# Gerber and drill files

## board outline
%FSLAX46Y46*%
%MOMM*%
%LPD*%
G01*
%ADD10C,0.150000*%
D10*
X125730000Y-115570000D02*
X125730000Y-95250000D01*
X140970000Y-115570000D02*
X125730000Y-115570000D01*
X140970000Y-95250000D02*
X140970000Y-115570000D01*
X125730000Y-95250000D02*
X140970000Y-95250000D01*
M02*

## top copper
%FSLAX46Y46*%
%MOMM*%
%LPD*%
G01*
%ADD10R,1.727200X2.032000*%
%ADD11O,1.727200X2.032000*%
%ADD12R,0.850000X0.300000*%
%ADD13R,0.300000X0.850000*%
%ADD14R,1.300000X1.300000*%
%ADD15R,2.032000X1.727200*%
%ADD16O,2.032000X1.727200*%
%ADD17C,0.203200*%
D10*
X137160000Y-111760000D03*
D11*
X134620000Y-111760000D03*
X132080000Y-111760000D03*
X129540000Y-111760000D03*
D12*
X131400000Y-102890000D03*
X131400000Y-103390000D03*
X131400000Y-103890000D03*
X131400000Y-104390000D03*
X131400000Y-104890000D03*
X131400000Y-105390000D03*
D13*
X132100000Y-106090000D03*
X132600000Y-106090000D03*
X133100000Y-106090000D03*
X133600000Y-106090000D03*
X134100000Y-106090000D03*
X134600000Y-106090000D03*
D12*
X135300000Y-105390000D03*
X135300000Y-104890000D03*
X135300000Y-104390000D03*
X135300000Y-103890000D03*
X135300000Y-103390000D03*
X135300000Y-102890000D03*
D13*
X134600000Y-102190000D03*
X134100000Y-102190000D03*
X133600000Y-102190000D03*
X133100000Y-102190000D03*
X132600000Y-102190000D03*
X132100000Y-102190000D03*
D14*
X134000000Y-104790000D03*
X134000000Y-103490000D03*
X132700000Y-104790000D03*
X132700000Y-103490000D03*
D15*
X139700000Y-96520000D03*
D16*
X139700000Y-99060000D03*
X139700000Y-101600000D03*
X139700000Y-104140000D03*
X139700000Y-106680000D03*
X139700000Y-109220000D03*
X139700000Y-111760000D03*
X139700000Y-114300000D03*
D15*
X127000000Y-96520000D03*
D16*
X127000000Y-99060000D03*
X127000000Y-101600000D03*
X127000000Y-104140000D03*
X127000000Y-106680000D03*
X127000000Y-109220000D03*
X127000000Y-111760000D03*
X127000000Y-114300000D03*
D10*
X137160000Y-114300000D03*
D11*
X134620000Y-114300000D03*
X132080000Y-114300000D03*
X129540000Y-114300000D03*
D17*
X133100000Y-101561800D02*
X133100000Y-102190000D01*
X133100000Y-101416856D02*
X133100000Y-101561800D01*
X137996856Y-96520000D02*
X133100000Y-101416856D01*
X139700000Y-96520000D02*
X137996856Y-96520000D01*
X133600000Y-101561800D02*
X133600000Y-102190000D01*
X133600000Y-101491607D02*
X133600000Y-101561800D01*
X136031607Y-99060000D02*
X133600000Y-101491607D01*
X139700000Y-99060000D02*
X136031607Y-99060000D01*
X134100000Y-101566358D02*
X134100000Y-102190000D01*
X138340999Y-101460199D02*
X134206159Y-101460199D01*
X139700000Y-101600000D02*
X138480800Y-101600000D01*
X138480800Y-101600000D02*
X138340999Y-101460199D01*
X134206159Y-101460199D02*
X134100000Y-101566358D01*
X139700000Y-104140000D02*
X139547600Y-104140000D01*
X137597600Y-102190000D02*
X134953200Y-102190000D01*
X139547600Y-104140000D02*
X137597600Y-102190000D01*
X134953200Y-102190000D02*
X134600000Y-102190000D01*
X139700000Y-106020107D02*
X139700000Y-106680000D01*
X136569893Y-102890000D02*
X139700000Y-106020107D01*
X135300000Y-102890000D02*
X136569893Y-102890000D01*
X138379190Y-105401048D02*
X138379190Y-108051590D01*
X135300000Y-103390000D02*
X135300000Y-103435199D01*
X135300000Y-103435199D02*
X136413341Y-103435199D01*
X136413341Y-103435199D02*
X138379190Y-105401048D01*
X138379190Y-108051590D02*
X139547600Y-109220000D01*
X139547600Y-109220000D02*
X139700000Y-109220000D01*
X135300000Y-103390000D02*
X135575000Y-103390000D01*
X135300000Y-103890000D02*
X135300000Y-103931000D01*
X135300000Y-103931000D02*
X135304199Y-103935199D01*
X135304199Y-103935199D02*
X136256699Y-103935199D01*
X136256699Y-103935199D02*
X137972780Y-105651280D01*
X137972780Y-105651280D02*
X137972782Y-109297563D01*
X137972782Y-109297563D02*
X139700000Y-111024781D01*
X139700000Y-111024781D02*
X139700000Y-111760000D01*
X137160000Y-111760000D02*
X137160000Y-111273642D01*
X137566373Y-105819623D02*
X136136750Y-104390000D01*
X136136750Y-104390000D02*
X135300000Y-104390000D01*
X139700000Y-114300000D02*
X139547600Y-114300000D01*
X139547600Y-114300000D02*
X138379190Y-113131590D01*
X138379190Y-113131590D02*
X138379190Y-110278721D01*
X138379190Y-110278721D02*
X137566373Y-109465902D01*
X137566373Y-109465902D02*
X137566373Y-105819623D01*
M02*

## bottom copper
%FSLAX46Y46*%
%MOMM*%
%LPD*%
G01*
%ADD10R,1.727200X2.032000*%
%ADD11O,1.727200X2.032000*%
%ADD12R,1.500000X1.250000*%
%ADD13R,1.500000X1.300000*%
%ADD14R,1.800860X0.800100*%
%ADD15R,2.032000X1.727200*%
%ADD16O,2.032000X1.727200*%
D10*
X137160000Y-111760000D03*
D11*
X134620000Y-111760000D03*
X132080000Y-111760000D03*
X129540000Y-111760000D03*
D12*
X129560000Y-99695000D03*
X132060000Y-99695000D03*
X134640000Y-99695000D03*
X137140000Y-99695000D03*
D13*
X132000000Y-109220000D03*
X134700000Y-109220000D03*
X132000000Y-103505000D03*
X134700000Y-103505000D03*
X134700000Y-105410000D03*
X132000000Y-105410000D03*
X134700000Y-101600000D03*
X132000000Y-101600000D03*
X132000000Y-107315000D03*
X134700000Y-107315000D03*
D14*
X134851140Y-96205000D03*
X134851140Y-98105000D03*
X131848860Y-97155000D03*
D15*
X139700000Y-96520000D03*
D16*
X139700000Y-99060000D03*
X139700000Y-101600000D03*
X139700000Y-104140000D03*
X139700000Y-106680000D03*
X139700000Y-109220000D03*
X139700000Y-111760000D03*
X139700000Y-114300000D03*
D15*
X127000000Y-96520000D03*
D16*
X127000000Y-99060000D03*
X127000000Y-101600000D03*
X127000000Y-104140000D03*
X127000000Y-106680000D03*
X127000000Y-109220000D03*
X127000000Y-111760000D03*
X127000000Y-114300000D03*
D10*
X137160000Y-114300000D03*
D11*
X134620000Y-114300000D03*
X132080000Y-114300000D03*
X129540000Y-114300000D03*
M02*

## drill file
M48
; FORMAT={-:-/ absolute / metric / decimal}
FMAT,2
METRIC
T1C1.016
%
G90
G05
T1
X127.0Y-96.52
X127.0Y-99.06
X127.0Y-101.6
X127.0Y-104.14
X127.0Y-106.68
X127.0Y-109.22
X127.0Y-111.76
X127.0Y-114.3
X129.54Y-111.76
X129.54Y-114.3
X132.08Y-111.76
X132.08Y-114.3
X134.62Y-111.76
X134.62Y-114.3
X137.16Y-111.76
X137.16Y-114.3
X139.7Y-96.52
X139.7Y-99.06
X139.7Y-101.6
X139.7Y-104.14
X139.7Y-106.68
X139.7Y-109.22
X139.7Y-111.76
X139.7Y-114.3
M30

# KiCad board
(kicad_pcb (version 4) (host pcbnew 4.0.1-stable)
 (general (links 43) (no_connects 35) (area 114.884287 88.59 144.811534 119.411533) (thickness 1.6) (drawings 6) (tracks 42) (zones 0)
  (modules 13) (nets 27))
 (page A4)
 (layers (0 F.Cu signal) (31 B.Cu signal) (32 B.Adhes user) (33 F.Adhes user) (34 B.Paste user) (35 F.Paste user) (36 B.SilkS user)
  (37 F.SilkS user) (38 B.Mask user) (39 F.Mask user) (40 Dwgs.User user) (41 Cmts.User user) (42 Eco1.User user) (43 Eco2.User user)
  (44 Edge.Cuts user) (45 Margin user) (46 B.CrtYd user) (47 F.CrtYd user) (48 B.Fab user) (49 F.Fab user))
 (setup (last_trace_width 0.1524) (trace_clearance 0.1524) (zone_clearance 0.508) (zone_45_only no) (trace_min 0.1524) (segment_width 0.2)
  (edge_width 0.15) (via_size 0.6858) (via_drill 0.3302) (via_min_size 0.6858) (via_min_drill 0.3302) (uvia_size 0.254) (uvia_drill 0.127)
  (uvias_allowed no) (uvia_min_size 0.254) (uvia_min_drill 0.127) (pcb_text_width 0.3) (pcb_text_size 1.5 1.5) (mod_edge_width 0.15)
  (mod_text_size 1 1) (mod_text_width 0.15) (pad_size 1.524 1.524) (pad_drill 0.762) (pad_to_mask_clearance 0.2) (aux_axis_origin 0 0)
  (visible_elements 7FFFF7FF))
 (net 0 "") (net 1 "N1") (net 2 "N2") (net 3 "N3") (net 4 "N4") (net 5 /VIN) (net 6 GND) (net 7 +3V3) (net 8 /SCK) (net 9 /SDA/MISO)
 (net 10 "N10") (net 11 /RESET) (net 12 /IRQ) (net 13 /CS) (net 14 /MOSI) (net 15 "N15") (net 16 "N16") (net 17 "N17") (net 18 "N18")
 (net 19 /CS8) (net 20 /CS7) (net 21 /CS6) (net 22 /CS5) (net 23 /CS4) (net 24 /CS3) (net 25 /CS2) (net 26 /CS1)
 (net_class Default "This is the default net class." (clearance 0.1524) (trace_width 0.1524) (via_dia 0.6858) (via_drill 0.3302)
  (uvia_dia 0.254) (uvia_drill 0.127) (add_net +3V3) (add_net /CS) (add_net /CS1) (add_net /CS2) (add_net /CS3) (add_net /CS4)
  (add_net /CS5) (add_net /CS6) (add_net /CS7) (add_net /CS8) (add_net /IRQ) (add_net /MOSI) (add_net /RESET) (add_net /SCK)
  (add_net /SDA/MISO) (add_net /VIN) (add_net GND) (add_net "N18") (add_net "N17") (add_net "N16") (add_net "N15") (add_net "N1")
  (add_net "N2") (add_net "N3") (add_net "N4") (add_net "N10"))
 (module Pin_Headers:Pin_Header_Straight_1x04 (layer F.Cu) (at 137.16 111.76 270)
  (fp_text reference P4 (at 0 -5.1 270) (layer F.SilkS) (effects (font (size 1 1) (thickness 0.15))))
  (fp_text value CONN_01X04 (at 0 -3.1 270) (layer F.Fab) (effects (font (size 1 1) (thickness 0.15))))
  (pad 1 thru_hole rect (at 0 0 270) (size 2.032 1.7272) (drill 1.016) (layers *.Cu *.Mask F.SilkS) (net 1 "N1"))
  (pad 2 thru_hole oval (at 0 2.54 270) (size 2.032 1.7272) (drill 1.016) (layers *.Cu *.Mask F.SilkS) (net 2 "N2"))
  (pad 3 thru_hole oval (at 0 5.08 270) (size 2.032 1.7272) (drill 1.016) (layers *.Cu *.Mask F.SilkS) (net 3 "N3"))
  (pad 4 thru_hole oval (at 0 7.62 270) (size 2.032 1.7272) (drill 1.016) (layers *.Cu *.Mask F.SilkS) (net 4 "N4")))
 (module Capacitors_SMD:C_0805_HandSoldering (layer B.Cu) (at 130.81 99.695)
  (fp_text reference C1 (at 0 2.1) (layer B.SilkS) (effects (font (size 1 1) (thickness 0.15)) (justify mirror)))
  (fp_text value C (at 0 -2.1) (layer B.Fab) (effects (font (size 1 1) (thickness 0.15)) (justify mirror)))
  (pad 1 smd rect (at -1.25 0) (size 1.5 1.25) (layers B.Cu B.Paste B.Mask) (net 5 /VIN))
  (pad 2 smd rect (at 1.25 0) (size 1.5 1.25) (layers B.Cu B.Paste B.Mask) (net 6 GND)))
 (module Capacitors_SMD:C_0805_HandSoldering (layer B.Cu) (at 135.89 99.695)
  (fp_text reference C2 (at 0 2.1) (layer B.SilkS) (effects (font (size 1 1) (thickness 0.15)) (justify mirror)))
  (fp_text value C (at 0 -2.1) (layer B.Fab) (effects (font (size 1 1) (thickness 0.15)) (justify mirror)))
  (pad 1 smd rect (at -1.25 0) (size 1.5 1.25) (layers B.Cu B.Paste B.Mask) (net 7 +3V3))
  (pad 2 smd rect (at 1.25 0) (size 1.5 1.25) (layers B.Cu B.Paste B.Mask) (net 6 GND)))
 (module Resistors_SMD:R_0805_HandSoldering (layer B.Cu) (at 133.35 109.22)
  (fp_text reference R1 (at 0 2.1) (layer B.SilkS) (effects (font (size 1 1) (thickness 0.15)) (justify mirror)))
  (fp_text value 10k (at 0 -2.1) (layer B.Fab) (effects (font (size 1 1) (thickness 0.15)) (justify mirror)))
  (pad 1 smd rect (at -1.35 0) (size 1.5 1.3) (layers B.Cu B.Paste B.Mask) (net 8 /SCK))
  (pad 2 smd rect (at 1.35 0) (size 1.5 1.3) (layers B.Cu B.Paste B.Mask) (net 7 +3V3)))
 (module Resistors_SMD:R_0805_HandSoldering (layer B.Cu) (at 133.35 103.505)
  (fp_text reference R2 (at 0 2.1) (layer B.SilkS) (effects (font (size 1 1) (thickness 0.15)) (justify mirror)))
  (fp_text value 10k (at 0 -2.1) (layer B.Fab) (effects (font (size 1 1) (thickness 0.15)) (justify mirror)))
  (pad 1 smd rect (at -1.35 0) (size 1.5 1.3) (layers B.Cu B.Paste B.Mask) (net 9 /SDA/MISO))
  (pad 2 smd rect (at 1.35 0) (size 1.5 1.3) (layers B.Cu B.Paste B.Mask) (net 7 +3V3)))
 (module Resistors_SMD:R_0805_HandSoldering (layer B.Cu) (at 133.35 105.41 180)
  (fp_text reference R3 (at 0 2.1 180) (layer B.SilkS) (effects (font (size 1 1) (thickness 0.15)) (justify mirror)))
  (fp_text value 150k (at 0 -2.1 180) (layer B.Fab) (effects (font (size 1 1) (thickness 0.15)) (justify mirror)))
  (pad 1 smd rect (at -1.35 0 180) (size 1.5 1.3) (layers B.Cu B.Paste B.Mask) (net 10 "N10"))
  (pad 2 smd rect (at 1.35 0 180) (size 1.5 1.3) (layers B.Cu B.Paste B.Mask) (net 6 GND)))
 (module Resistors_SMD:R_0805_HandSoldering (layer B.Cu) (at 133.35 101.6 180)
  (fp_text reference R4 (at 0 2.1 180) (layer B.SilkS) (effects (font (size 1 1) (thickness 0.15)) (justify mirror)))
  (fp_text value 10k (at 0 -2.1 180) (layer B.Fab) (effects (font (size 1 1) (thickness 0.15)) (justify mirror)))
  (pad 1 smd rect (at -1.35 0 180) (size 1.5 1.3) (layers B.Cu B.Paste B.Mask) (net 6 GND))
  (pad 2 smd rect (at 1.35 0 180) (size 1.5 1.3) (layers B.Cu B.Paste B.Mask) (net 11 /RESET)))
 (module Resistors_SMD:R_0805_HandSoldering (layer B.Cu) (at 133.35 107.315)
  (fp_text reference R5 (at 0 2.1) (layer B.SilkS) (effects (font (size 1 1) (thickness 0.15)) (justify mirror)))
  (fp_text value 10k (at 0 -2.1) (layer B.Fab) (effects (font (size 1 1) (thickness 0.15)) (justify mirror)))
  (pad 1 smd rect (at -1.35 0) (size 1.5 1.3) (layers B.Cu B.Paste B.Mask) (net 7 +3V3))
  (pad 2 smd rect (at 1.35 0) (size 1.5 1.3) (layers B.Cu B.Paste B.Mask) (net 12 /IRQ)))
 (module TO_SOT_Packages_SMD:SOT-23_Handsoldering (layer B.Cu) (at 133.35 97.155 270)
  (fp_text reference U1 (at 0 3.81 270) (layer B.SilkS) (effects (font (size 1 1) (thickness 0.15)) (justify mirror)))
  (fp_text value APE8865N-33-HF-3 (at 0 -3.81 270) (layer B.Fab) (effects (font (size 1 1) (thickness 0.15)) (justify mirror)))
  (pad 1 smd rect (at -0.95 -1.50114 270) (size 0.8001 1.80086) (layers B.Cu B.Paste B.Mask) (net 6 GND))
  (pad 2 smd rect (at 0.95 -1.50114 270) (size 0.8001 1.80086) (layers B.Cu B.Paste B.Mask) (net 7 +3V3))
  (pad 3 smd rect (at 0 1.50114 270) (size 0.8001 1.80086) (layers B.Cu B.Paste B.Mask) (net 5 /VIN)))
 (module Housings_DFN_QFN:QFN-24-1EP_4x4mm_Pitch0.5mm (layer F.Cu) (at 133.35 104.14)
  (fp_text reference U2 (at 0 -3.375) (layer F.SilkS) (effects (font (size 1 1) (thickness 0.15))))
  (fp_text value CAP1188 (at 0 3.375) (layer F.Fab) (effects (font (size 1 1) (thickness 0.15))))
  (pad 1 smd rect (at -1.95 -1.25) (size 0.85 0.3) (layers F.Cu F.Paste F.Mask) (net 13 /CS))
  (pad 2 smd rect (at -1.95 -0.75) (size 0.85 0.3) (layers F.Cu F.Paste F.Mask) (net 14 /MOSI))
  (pad 3 smd rect (at -1.95 -0.25) (size 0.85 0.3) (layers F.Cu F.Paste F.Mask) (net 9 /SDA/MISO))
  (pad 4 smd rect (at -1.95 0.25) (size 0.85 0.3) (layers F.Cu F.Paste F.Mask) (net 8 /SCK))
  (pad 5 smd rect (at -1.95 0.75) (size 0.85 0.3) (layers F.Cu F.Paste F.Mask) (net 4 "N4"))
  (pad 6 smd rect (at -1.95 1.25) (size 0.85 0.3) (layers F.Cu F.Paste F.Mask) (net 3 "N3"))
  (pad 7 smd rect (at -1.25 1.95 90) (size 0.85 0.3) (layers F.Cu F.Paste F.Mask) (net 2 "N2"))
  (pad 8 smd rect (at -0.75 1.95 90) (size 0.85 0.3) (layers F.Cu F.Paste F.Mask) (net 1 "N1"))
  (pad 9 smd rect (at -0.25 1.95 90) (size 0.85 0.3) (layers F.Cu F.Paste F.Mask) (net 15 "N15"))
  (pad 10 smd rect (at 0.25 1.95 90) (size 0.85 0.3) (layers F.Cu F.Paste F.Mask) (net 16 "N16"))
  (pad 11 smd rect (at 0.75 1.95 90) (size 0.85 0.3) (layers F.Cu F.Paste F.Mask) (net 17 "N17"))
  (pad 12 smd rect (at 1.25 1.95 90) (size 0.85 0.3) (layers F.Cu F.Paste F.Mask) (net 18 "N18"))
  (pad 13 smd rect (at 1.95 1.25) (size 0.85 0.3) (layers F.Cu F.Paste F.Mask) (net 12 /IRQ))
  (pad 14 smd rect (at 1.95 0.75) (size 0.85 0.3) (layers F.Cu F.Paste F.Mask) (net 10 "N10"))
  (pad 15 smd rect (at 1.95 0.25) (size 0.85 0.3) (layers F.Cu F.Paste F.Mask) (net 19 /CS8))
  (pad 16 smd rect (at 1.95 -0.25) (size 0.85 0.3) (layers F.Cu F.Paste F.Mask) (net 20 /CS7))
  (pad 17 smd rect (at 1.95 -0.75) (size 0.85 0.3) (layers F.Cu F.Paste F.Mask) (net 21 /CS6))
  (pad 18 smd rect (at 1.95 -1.25) (size 0.85 0.3) (layers F.Cu F.Paste F.Mask) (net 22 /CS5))
  (pad 19 smd rect (at 1.25 -1.95 90) (size 0.85 0.3) (layers F.Cu F.Paste F.Mask) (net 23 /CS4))
  (pad 20 smd rect (at 0.75 -1.95 90) (size 0.85 0.3) (layers F.Cu F.Paste F.Mask) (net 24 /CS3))
  (pad 21 smd rect (at 0.25 -1.95 90) (size 0.85 0.3) (layers F.Cu F.Paste F.Mask) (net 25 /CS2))
  (pad 22 smd rect (at -0.25 -1.95 90) (size 0.85 0.3) (layers F.Cu F.Paste F.Mask) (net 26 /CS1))
  (pad 23 smd rect (at -0.75 -1.95 90) (size 0.85 0.3) (layers F.Cu F.Paste F.Mask) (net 7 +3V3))
  (pad 24 smd rect (at -1.25 -1.95 90) (size 0.85 0.3) (layers F.Cu F.Paste F.Mask) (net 11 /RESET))
  (pad 25 smd rect (at 0.65 0.65) (size 1.3 1.3) (layers F.Cu F.Paste F.Mask) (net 6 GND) (solder_paste_margin_ratio -0.2))
  (pad 25 smd rect (at 0.65 -0.65) (size 1.3 1.3) (layers F.Cu F.Paste F.Mask) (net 6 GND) (solder_paste_margin_ratio -0.2))
  (pad 25 smd rect (at -0.65 0.65) (size 1.3 1.3) (layers F.Cu F.Paste F.Mask) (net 6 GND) (solder_paste_margin_ratio -0.2))
  (pad 25 smd rect (at -0.65 -0.65) (size 1.3 1.3) (layers F.Cu F.Paste F.Mask) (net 6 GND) (solder_paste_margin_ratio -0.2)))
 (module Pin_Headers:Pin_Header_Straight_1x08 (layer B.Cu) (at 139.7 96.52 180)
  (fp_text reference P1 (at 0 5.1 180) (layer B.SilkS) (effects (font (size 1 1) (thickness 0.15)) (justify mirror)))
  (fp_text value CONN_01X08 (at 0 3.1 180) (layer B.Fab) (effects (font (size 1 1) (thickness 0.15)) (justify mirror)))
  (pad 1 thru_hole rect (at 0 0 180) (size 2.032 1.7272) (drill 1.016) (layers *.Cu *.Mask B.SilkS) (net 26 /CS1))
  (pad 2 thru_hole oval (at 0 -2.54 180) (size 2.032 1.7272) (drill 1.016) (layers *.Cu *.Mask B.SilkS) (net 25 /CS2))
  (pad 3 thru_hole oval (at 0 -5.08 180) (size 2.032 1.7272) (drill 1.016) (layers *.Cu *.Mask B.SilkS) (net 24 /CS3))
  (pad 4 thru_hole oval (at 0 -7.62 180) (size 2.032 1.7272) (drill 1.016) (layers *.Cu *.Mask B.SilkS) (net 23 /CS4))
  (pad 5 thru_hole oval (at 0 -10.16 180) (size 2.032 1.7272) (drill 1.016) (layers *.Cu *.Mask B.SilkS) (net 22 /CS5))
  (pad 6 thru_hole oval (at 0 -12.7 180) (size 2.032 1.7272) (drill 1.016) (layers *.Cu *.Mask B.SilkS) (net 21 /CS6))
  (pad 7 thru_hole oval (at 0 -15.24 180) (size 2.032 1.7272) (drill 1.016) (layers *.Cu *.Mask B.SilkS) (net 20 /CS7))
  (pad 8 thru_hole oval (at 0 -17.78 180) (size 2.032 1.7272) (drill 1.016) (layers *.Cu *.Mask B.SilkS) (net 19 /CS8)))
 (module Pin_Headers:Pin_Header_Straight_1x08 (layer B.Cu) (at 127 96.52 180)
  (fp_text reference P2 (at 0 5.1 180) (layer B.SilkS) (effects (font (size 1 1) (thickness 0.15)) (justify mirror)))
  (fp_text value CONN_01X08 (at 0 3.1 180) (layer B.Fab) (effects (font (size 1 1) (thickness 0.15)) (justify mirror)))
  (pad 1 thru_hole rect (at 0 0 180) (size 2.032 1.7272) (drill 1.016) (layers *.Cu *.Mask B.SilkS) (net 9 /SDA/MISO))
  (pad 2 thru_hole oval (at 0 -2.54 180) (size 2.032 1.7272) (drill 1.016) (layers *.Cu *.Mask B.SilkS) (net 8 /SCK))
  (pad 3 thru_hole oval (at 0 -5.08 180) (size 2.032 1.7272) (drill 1.016) (layers *.Cu *.Mask B.SilkS) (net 5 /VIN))
  (pad 4 thru_hole oval (at 0 -7.62 180) (size 2.032 1.7272) (drill 1.016) (layers *.Cu *.Mask B.SilkS) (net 6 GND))
  (pad 5 thru_hole oval (at 0 -10.16 180) (size 2.032 1.7272) (drill 1.016) (layers *.Cu *.Mask B.SilkS) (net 14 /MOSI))
  (pad 6 thru_hole oval (at 0 -12.7 180) (size 2.032 1.7272) (drill 1.016) (layers *.Cu *.Mask B.SilkS) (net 13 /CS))
  (pad 7 thru_hole oval (at 0 -15.24 180) (size 2.032 1.7272) (drill 1.016) (layers *.Cu *.Mask B.SilkS) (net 11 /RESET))
  (pad 8 thru_hole oval (at 0 -17.78 180) (size 2.032 1.7272) (drill 1.016) (layers *.Cu *.Mask B.SilkS) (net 12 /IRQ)))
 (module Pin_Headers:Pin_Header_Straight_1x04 (layer F.Cu) (at 137.16 114.3 270)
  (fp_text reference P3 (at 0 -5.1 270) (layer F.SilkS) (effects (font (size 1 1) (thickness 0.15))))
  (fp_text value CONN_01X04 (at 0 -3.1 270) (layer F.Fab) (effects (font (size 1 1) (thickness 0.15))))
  (pad 1 thru_hole rect (at 0 0 270) (size 2.032 1.7272) (drill 1.016) (layers *.Cu *.Mask F.SilkS) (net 18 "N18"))
  (pad 2 thru_hole oval (at 0 2.54 270) (size 2.032 1.7272) (drill 1.016) (layers *.Cu *.Mask F.SilkS) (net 17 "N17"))
  (pad 3 thru_hole oval (at 0 5.08 270) (size 2.032 1.7272) (drill 1.016) (layers *.Cu *.Mask F.SilkS) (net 16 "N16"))
  (pad 4 thru_hole oval (at 0 7.62 270) (size 2.032 1.7272) (drill 1.016) (layers *.Cu *.Mask F.SilkS) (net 15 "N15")))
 (gr_line (start 125.73 115.57) (end 125.73 95.25) (angle 90) (layer Edge.Cuts) (width 0.15))
 (gr_line (start 140.97 115.57) (end 125.73 115.57) (angle 90) (layer Edge.Cuts) (width 0.15))
 (gr_line (start 140.97 95.25) (end 140.97 115.57) (angle 90) (layer Edge.Cuts) (width 0.15))
 (gr_line (start 125.73 95.25) (end 140.97 95.25) (angle 90) (layer Edge.Cuts) (width 0.15))
 (segment (start 133.1 101.5618) (end 133.1 102.19) (width 0.2032) (layer F.Cu) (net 26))
 (segment (start 133.1 101.416856) (end 133.1 101.5618) (width 0.2032) (layer F.Cu) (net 26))
 (segment (start 137.996856 96.52) (end 133.1 101.416856) (width 0.2032) (layer F.Cu) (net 26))
 (segment (start 139.7 96.52) (end 137.996856 96.52) (width 0.2032) (layer F.Cu) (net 26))
 (segment (start 133.6 101.5618) (end 133.6 102.19) (width 0.2032) (layer F.Cu) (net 25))
 (segment (start 133.6 101.491607) (end 133.6 101.5618) (width 0.2032) (layer F.Cu) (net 25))
 (segment (start 136.031607 99.06) (end 133.6 101.491607) (width 0.2032) (layer F.Cu) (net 25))
 (segment (start 139.7 99.06) (end 136.031607 99.06) (width 0.2032) (layer F.Cu) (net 25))
 (segment (start 134.1 101.566358) (end 134.1 102.19) (width 0.2032) (layer F.Cu) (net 24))
 (segment (start 138.340999 101.460199) (end 134.206159 101.460199) (width 0.2032) (layer F.Cu) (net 24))
 (segment (start 139.7 101.6) (end 138.4808 101.6) (width 0.2032) (layer F.Cu) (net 24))
 (segment (start 138.4808 101.6) (end 138.340999 101.460199) (width 0.2032) (layer F.Cu) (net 24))
 (segment (start 134.206159 101.460199) (end 134.1 101.566358) (width 0.2032) (layer F.Cu) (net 24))
 (segment (start 139.7 104.14) (end 139.5476 104.14) (width 0.2032) (layer F.Cu) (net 23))
 (segment (start 137.5976 102.19) (end 134.9532 102.19) (width 0.2032) (layer F.Cu) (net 23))
 (segment (start 139.5476 104.14) (end 137.5976 102.19) (width 0.2032) (layer F.Cu) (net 23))
 (segment (start 134.9532 102.19) (end 134.6 102.19) (width 0.2032) (layer F.Cu) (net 23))
 (segment (start 139.7 106.020107) (end 139.7 106.68) (width 0.2032) (layer F.Cu) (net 22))
 (segment (start 136.569893 102.89) (end 139.7 106.020107) (width 0.2032) (layer F.Cu) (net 22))
 (segment (start 135.3 102.89) (end 136.569893 102.89) (width 0.2032) (layer F.Cu) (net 22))
 (segment (start 138.37919 105.401048) (end 138.37919 108.05159) (width 0.2032) (layer F.Cu) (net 21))
 (segment (start 135.3 103.39) (end 135.3 103.435199) (width 0.2032) (layer F.Cu) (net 21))
 (segment (start 135.3 103.435199) (end 136.413341 103.435199) (width 0.2032) (layer F.Cu) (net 21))
 (segment (start 136.413341 103.435199) (end 138.37919 105.401048) (width 0.2032) (layer F.Cu) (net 21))
 (segment (start 138.37919 108.05159) (end 139.5476 109.22) (width 0.2032) (layer F.Cu) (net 21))
 (segment (start 139.5476 109.22) (end 139.7 109.22) (width 0.2032) (layer F.Cu) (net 21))
 (segment (start 135.3 103.39) (end 135.575 103.39) (width 0.2032) (layer F.Cu) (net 21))
 (segment (start 135.3 103.89) (end 135.3 103.931) (width 0.2032) (layer F.Cu) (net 20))
 (segment (start 135.3 103.931) (end 135.304199 103.935199) (width 0.2032) (layer F.Cu) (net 20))
 (segment (start 135.304199 103.935199) (end 136.256699 103.935199) (width 0.2032) (layer F.Cu) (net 20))
 (segment (start 136.256699 103.935199) (end 137.97278 105.65128) (width 0.2032) (layer F.Cu) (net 20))
 (segment (start 137.97278 105.65128) (end 137.972782 109.297563) (width 0.2032) (layer F.Cu) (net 20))
 (segment (start 137.972782 109.297563) (end 139.7 111.024781) (width 0.2032) (layer F.Cu) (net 20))
 (segment (start 139.7 111.024781) (end 139.7 111.76) (width 0.2032) (layer F.Cu) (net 20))
 (segment (start 137.16 111.76) (end 137.16 111.273642) (width 0.2032) (layer F.Cu) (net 1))
 (segment (start 137.566373 105.819623) (end 136.13675 104.39) (width 0.2032) (layer F.Cu) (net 19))
 (segment (start 136.13675 104.39) (end 135.3 104.39) (width 0.2032) (layer F.Cu) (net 19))
 (segment (start 139.7 114.3) (end 139.5476 114.3) (width 0.2032) (layer F.Cu) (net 19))
 (segment (start 139.5476 114.3) (end 138.37919 113.13159) (width 0.2032) (layer F.Cu) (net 19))
 (segment (start 138.37919 113.13159) (end 138.37919 110.278721) (width 0.2032) (layer F.Cu) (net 19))
 (segment (start 138.37919 110.278721) (end 137.566373 109.465902) (width 0.2032) (layer F.Cu) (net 19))
 (segment (start 137.566373 109.465902) (end 137.566373 105.819623) (width 0.2032) (layer F.Cu) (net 19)))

